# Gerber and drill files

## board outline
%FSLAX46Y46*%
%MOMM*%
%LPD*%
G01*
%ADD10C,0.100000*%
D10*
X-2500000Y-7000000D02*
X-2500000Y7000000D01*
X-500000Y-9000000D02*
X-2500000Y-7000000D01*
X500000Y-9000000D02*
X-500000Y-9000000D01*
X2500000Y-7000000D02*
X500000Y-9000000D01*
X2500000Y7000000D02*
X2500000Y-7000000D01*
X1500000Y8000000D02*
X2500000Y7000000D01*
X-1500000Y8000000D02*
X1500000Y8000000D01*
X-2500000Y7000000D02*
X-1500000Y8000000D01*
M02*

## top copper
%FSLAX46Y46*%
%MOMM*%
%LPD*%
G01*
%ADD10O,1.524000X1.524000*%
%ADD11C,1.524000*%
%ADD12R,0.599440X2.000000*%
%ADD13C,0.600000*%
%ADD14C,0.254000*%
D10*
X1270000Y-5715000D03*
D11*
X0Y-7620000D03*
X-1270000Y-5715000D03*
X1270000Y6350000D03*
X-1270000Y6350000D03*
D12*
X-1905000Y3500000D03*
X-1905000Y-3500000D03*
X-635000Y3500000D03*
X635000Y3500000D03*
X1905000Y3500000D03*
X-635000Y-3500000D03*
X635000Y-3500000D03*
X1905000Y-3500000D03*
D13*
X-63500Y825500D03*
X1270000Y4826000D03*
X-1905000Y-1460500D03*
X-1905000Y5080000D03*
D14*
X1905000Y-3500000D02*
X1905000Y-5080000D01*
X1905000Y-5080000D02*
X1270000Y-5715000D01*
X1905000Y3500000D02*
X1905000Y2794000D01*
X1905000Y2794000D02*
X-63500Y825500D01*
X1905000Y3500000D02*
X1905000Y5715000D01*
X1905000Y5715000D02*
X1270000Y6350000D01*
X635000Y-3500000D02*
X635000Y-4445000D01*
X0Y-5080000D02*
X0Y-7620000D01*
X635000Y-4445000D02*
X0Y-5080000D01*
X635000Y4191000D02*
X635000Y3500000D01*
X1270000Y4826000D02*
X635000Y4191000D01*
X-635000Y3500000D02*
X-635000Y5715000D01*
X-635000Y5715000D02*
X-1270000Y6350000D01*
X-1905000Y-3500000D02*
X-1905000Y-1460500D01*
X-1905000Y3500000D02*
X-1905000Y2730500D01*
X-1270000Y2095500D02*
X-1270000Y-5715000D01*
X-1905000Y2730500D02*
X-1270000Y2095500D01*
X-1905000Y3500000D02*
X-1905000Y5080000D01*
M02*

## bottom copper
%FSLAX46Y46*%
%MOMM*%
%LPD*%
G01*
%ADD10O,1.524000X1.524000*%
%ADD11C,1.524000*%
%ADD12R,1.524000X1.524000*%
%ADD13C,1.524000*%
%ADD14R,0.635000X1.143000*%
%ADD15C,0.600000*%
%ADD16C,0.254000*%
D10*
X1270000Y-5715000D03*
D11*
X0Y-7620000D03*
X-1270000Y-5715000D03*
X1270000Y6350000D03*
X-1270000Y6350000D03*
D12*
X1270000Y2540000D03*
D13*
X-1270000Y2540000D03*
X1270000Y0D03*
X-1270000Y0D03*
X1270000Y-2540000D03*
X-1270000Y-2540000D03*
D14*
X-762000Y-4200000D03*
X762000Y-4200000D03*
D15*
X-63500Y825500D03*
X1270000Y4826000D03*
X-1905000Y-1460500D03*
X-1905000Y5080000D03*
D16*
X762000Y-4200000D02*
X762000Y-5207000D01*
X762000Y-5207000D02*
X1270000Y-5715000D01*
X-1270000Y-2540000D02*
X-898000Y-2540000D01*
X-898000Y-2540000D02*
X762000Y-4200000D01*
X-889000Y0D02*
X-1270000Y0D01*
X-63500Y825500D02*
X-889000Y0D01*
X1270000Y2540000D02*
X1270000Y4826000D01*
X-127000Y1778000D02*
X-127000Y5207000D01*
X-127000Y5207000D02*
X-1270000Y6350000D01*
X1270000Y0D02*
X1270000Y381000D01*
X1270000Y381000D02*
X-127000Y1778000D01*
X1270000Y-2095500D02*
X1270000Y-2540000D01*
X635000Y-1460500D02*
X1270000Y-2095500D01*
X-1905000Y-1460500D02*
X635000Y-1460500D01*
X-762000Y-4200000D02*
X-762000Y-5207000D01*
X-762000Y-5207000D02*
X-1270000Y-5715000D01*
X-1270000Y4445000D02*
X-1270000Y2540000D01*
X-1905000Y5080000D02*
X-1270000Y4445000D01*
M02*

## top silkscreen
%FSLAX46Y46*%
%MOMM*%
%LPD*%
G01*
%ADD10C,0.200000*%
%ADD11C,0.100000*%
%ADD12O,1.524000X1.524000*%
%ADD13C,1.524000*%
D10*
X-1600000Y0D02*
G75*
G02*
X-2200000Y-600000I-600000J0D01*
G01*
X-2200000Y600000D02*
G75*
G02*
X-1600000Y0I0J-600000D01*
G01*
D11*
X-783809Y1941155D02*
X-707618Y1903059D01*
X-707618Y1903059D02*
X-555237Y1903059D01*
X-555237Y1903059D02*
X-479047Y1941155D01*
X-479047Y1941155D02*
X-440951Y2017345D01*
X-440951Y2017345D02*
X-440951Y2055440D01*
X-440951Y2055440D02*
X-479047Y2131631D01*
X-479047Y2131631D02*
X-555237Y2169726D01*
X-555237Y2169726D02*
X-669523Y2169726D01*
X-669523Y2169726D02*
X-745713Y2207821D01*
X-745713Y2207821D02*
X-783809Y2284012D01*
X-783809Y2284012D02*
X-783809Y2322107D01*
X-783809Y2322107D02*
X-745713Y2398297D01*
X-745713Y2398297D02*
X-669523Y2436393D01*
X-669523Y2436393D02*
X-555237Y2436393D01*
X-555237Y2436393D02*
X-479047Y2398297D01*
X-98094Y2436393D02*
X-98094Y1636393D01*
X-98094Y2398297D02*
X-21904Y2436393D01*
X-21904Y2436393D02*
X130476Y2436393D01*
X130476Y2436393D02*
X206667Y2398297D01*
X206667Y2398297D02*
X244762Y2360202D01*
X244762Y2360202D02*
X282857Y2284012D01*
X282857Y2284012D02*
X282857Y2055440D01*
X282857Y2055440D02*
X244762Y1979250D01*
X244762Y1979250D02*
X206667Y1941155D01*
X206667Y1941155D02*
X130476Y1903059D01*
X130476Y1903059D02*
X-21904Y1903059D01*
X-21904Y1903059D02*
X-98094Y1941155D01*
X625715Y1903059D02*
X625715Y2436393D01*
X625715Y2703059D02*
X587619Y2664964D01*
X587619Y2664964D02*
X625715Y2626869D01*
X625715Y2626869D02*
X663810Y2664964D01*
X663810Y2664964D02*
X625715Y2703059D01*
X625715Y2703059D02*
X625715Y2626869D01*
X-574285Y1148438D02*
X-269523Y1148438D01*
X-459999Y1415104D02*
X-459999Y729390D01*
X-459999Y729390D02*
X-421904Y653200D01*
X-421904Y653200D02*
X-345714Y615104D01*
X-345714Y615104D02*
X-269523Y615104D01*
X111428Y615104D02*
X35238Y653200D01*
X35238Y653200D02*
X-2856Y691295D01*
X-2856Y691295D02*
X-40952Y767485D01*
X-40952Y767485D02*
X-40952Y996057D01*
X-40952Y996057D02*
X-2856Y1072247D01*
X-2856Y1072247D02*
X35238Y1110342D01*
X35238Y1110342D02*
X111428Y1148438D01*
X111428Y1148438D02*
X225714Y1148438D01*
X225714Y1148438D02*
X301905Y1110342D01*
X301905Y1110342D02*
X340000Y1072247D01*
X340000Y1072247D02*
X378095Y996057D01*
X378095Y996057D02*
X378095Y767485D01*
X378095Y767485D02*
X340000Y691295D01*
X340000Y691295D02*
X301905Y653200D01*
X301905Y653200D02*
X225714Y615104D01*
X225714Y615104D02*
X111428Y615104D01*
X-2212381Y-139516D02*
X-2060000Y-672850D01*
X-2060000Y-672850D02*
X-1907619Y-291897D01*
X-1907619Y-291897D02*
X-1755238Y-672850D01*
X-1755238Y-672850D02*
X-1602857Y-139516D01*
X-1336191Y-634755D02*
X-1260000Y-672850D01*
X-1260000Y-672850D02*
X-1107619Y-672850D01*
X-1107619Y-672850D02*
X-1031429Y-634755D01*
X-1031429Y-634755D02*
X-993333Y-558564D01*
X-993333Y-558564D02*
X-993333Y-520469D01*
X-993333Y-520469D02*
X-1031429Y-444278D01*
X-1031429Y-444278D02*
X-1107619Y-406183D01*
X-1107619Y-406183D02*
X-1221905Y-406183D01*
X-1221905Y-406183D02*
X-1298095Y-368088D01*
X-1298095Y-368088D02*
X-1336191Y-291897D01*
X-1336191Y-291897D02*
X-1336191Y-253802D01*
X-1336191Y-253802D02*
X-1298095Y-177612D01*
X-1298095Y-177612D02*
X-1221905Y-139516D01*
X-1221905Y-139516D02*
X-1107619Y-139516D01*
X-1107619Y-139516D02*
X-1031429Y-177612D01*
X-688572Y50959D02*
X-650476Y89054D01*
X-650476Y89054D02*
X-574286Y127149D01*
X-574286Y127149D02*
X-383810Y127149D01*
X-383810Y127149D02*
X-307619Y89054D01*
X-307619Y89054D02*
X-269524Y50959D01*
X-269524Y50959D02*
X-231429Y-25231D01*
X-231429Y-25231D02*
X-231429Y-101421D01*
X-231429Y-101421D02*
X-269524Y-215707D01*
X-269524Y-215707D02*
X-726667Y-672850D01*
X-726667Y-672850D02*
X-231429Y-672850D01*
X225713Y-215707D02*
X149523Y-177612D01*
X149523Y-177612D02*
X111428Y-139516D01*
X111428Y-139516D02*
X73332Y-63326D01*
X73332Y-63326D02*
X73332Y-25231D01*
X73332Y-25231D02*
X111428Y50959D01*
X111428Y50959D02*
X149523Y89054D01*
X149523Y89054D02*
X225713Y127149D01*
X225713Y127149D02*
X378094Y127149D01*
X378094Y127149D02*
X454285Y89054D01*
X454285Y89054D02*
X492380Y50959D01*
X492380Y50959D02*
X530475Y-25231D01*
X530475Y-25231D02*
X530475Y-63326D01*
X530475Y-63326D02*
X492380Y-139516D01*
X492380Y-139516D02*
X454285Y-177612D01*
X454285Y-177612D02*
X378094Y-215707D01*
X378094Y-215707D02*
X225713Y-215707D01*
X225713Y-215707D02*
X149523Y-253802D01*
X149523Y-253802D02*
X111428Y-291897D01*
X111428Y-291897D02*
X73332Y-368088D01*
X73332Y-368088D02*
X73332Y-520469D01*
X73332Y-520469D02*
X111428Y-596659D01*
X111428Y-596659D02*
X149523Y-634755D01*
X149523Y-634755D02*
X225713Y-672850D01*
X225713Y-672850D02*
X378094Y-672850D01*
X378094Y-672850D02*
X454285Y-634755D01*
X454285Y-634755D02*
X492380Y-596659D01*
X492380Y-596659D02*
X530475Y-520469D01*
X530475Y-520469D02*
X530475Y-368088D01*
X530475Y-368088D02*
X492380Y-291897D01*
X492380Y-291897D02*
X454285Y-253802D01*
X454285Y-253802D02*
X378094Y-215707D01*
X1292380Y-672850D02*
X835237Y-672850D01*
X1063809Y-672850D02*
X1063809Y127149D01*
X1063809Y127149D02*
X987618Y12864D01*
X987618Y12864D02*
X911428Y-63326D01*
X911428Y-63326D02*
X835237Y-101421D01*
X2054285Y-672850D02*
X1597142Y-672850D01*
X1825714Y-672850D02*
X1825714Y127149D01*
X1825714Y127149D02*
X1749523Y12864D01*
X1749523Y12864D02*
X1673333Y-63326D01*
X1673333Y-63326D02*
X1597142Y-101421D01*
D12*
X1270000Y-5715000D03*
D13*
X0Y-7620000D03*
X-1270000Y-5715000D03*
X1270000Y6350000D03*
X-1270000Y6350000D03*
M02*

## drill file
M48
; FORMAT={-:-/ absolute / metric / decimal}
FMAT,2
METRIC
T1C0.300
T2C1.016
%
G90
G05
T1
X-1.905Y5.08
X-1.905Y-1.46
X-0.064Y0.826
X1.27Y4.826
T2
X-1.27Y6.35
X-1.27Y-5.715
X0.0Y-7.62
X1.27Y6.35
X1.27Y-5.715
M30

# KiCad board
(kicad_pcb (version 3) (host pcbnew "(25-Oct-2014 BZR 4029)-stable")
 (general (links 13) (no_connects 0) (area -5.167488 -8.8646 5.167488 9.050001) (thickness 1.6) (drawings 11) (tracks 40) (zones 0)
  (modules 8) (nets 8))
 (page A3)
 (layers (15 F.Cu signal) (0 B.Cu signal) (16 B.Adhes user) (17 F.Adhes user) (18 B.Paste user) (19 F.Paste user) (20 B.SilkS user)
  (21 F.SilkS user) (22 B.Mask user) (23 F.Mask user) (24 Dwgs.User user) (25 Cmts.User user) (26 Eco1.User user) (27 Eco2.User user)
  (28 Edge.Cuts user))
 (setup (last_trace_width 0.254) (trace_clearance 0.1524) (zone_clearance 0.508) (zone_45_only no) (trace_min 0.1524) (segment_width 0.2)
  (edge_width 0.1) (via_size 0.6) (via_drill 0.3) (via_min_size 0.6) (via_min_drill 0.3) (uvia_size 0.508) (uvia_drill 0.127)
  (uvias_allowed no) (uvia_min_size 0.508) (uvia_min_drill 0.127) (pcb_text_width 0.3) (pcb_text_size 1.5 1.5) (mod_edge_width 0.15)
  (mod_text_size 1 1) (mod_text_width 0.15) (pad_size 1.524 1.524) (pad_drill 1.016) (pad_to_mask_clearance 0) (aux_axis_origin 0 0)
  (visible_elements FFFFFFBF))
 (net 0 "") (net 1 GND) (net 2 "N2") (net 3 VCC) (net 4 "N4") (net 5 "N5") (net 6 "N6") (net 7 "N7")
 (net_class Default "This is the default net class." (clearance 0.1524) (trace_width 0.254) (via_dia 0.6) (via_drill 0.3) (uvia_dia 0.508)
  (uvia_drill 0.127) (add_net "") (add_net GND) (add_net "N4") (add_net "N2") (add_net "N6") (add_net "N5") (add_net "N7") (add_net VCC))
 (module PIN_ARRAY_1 (layer F.Cu) (at 1.27 5.715)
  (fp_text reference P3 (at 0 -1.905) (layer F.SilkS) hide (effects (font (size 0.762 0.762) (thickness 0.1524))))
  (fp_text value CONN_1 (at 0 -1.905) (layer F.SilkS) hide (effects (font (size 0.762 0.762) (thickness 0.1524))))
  (pad 1 thru_hole oval (at 0 0) (size 1.524 1.524) (drill 1.016) (layers *.Cu *.Mask F.SilkS) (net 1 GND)))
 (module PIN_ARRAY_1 (layer F.Cu) (at 0 7.62)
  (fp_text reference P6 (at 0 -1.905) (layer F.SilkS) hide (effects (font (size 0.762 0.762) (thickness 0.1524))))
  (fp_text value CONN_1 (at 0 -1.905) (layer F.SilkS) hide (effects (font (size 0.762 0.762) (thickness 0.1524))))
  (pad 1 thru_hole circle (at 0 0) (size 1.524 1.524) (drill 1.016) (layers *.Cu *.Mask F.SilkS) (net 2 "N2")))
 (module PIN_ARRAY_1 (layer F.Cu) (at -1.27 5.715)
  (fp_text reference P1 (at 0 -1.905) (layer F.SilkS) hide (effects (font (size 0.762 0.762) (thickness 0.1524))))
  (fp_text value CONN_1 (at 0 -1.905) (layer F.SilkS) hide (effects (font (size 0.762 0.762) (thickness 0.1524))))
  (pad 1 thru_hole circle (at 0 0) (size 1.524 1.524) (drill 1.016) (layers *.Cu *.Mask F.SilkS) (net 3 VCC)))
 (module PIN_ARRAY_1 (layer F.Cu) (at 1.27 -6.35)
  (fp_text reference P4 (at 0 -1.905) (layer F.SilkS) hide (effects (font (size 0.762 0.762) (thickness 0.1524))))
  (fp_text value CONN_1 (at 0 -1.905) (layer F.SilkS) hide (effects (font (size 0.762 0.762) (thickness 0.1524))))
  (pad 1 thru_hole circle (at 0 0) (size 1.524 1.524) (drill 1.016) (layers *.Cu *.Mask F.SilkS) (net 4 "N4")))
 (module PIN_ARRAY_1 (layer F.Cu) (at -1.27 -6.35)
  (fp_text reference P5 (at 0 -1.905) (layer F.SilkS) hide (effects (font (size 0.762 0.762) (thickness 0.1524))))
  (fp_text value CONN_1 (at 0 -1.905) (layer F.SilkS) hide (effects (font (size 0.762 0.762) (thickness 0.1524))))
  (pad 1 thru_hole circle (at 0 0) (size 1.524 1.524) (drill 1.016) (layers *.Cu *.Mask F.SilkS) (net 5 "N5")))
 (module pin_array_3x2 (layer B.Cu) (at 0 0 270)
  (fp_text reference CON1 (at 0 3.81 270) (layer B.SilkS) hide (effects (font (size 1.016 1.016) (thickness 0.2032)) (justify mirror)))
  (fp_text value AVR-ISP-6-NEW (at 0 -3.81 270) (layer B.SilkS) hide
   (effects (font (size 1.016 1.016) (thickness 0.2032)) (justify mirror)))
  (pad 1 smd rect (at -2.54 -1.27 270) (size 1.524 1.524) (layers B.Cu B.Paste B.Mask) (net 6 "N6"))
  (pad 2 smd circle (at -2.54 1.27 270) (size 1.524 1.524) (layers B.Cu B.Paste B.Mask) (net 3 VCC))
  (pad 3 smd circle (at 0 -1.27 270) (size 1.524 1.524) (layers B.Cu B.Paste B.Mask) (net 5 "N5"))
  (pad 4 smd circle (at 0 1.27 270) (size 1.524 1.524) (layers B.Cu B.Paste B.Mask) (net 4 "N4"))
  (pad 5 smd circle (at 2.54 -1.27 270) (size 1.524 1.524) (layers B.Cu B.Paste B.Mask) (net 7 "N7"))
  (pad 6 smd circle (at 2.54 1.27 270) (size 1.524 1.524) (layers B.Cu B.Paste B.Mask) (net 1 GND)))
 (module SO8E (layer F.Cu) (at 0 0)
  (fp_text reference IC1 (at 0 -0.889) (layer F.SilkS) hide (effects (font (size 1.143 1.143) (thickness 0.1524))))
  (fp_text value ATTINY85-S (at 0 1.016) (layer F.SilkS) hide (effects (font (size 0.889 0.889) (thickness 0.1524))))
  (pad 8 smd rect (at -1.905 -3.5) (size 0.59944 2) (layers F.Cu F.Paste F.Mask) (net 3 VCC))
  (pad 1 smd rect (at -1.905 3.5) (size 0.59944 2) (layers F.Cu F.Paste F.Mask) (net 7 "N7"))
  (pad 7 smd rect (at -0.635 -3.5) (size 0.59944 2) (layers F.Cu F.Paste F.Mask) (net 5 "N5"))
  (pad 6 smd rect (at 0.635 -3.5) (size 0.59944 2) (layers F.Cu F.Paste F.Mask) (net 6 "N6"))
  (pad 5 smd rect (at 1.905 -3.5) (size 0.59944 2) (layers F.Cu F.Paste F.Mask) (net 4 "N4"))
  (pad 2 smd rect (at -0.635 3.5) (size 0.59944 2) (layers F.Cu F.Paste F.Mask))
  (pad 3 smd rect (at 0.635 3.5) (size 0.59944 2) (layers F.Cu F.Paste F.Mask) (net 2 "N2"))
  (pad 4 smd rect (at 1.905 3.5) (size 0.59944 2) (layers F.Cu F.Paste F.Mask) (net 1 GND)))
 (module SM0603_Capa (layer B.Cu) (at 0 4.2)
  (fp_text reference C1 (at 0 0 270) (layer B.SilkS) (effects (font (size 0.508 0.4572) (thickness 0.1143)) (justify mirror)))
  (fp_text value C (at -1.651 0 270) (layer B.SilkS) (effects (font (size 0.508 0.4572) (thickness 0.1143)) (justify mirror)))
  (pad 1 smd rect (at -0.762 0) (size 0.635 1.143) (layers B.Cu B.Paste B.Mask) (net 3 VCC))
  (pad 2 smd rect (at 0.762 0) (size 0.635 1.143) (layers B.Cu B.Paste B.Mask) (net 1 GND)))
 (gr_arc (start -2.2 0) (end -1.6 0) (angle 90) (layer F.SilkS) (width 0.2))
 (gr_arc (start -2.2 0) (end -2.2 -0.6) (angle 90) (layer F.SilkS) (width 0.2))
 (gr_line (start -2.5 7) (end -2.5 -7) (angle 90) (layer Edge.Cuts) (width 0.1))
 (gr_line (start -0.5 9) (end -2.5 7) (angle 90) (layer Edge.Cuts) (width 0.1))
 (gr_line (start 0.5 9) (end -0.5 9) (angle 90) (layer Edge.Cuts) (width 0.1))
 (gr_line (start 2.5 7) (end 0.5 9) (angle 90) (layer Edge.Cuts) (width 0.1))
 (gr_line (start 2.5 -7) (end 2.5 7) (angle 90) (layer Edge.Cuts) (width 0.1))
 (gr_line (start 1.5 -8) (end 2.5 -7) (angle 90) (layer Edge.Cuts) (width 0.1))
 (gr_line (start -1.5 -8) (end 1.5 -8) (angle 90) (layer Edge.Cuts) (width 0.1))
 (gr_line (start -2.5 -7) (end -1.5 -8) (angle 90) (layer Edge.Cuts) (width 0.1))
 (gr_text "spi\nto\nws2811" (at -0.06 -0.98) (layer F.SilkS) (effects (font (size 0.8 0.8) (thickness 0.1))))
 (segment (start 0.762 4.2) (end 0.762 5.207) (width 0.254) (layer B.Cu) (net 1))
 (segment (start 0.762 5.207) (end 1.27 5.715) (width 0.254) (layer B.Cu) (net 1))
 (segment (start -1.27 2.54) (end -0.898 2.54) (width 0.254) (layer B.Cu) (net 1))
 (segment (start -0.898 2.54) (end 0.762 4.2) (width 0.254) (layer B.Cu) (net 1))
 (segment (start 1.905 3.5) (end 1.905 5.08) (width 0.254) (layer F.Cu) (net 1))
 (segment (start 1.905 5.08) (end 1.27 5.715) (width 0.254) (layer F.Cu) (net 1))
 (segment (start 1.905 -3.5) (end 1.905 -2.794) (width 0.254) (layer F.Cu) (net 4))
 (segment (start -0.889 0) (end -1.27 0) (width 0.254) (layer B.Cu) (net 4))
 (segment (start -0.0635 -0.8255) (end -0.889 0) (width 0.254) (layer B.Cu) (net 4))
 (via (at -0.0635 -0.8255) (size 0.6) (layers F.Cu B.Cu) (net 4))
 (segment (start 1.905 -2.794) (end -0.0635 -0.8255) (width 0.254) (layer F.Cu) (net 4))
 (segment (start 1.905 -3.5) (end 1.905 -5.715) (width 0.254) (layer F.Cu) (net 4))
 (segment (start 1.905 -5.715) (end 1.27 -6.35) (width 0.254) (layer F.Cu) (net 4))
 (segment (start 0.635 3.5) (end 0.635 4.445) (width 0.254) (layer F.Cu) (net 2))
 (segment (start 0 5.08) (end 0 7.62) (width 0.254) (layer F.Cu) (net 2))
 (segment (start 0.635 4.445) (end 0 5.08) (width 0.254) (layer F.Cu) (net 2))
 (segment (start 1.27 -2.54) (end 1.27 -4.826) (width 0.254) (layer B.Cu) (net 6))
 (segment (start 0.635 -4.191) (end 0.635 -3.5) (width 0.254) (layer F.Cu) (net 6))
 (segment (start 1.27 -4.826) (end 0.635 -4.191) (width 0.254) (layer F.Cu) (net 6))
 (via (at 1.27 -4.826) (size 0.6) (layers F.Cu B.Cu) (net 6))
 (segment (start -0.635 -3.5) (end -0.635 -5.715) (width 0.254) (layer F.Cu) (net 5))
 (segment (start -0.635 -5.715) (end -1.27 -6.35) (width 0.254) (layer F.Cu) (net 5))
 (segment (start -0.127 -1.778) (end -0.127 -5.207) (width 0.254) (layer B.Cu) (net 5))
 (segment (start -0.127 -5.207) (end -1.27 -6.35) (width 0.254) (layer B.Cu) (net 5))
 (segment (start 1.27 0) (end 1.27 -0.381) (width 0.254) (layer B.Cu) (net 5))
 (segment (start 1.27 -0.381) (end -0.127 -1.778) (width 0.254) (layer B.Cu) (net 5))
 (segment (start -1.905 3.5) (end -1.905 1.4605) (width 0.254) (layer F.Cu) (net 7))
 (segment (start 1.27 2.0955) (end 1.27 2.54) (width 0.254) (layer B.Cu) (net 7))
 (segment (start 0.635 1.4605) (end 1.27 2.0955) (width 0.254) (layer B.Cu) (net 7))
 (segment (start -1.905 1.4605) (end 0.635 1.4605) (width 0.254) (layer B.Cu) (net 7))
 (via (at -1.905 1.4605) (size 0.6) (layers F.Cu B.Cu) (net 7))
 (segment (start -0.762 4.2) (end -0.762 5.207) (width 0.254) (layer B.Cu) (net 3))
 (segment (start -0.762 5.207) (end -1.27 5.715) (width 0.254) (layer B.Cu) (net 3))
 (segment (start -1.905 -3.5) (end -1.905 -2.7305) (width 0.254) (layer F.Cu) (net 3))
 (segment (start -1.27 -2.0955) (end -1.27 5.715) (width 0.254) (layer F.Cu) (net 3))
 (segment (start -1.905 -2.7305) (end -1.27 -2.0955) (width 0.254) (layer F.Cu) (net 3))
 (segment (start -1.905 -3.5) (end -1.905 -5.08) (width 0.254) (layer F.Cu) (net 3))
 (segment (start -1.27 -4.445) (end -1.27 -2.54) (width 0.254) (layer B.Cu) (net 3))
 (segment (start -1.905 -5.08) (end -1.27 -4.445) (width 0.254) (layer B.Cu) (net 3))
 (via (at -1.905 -5.08) (size 0.6) (layers F.Cu B.Cu) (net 3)))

